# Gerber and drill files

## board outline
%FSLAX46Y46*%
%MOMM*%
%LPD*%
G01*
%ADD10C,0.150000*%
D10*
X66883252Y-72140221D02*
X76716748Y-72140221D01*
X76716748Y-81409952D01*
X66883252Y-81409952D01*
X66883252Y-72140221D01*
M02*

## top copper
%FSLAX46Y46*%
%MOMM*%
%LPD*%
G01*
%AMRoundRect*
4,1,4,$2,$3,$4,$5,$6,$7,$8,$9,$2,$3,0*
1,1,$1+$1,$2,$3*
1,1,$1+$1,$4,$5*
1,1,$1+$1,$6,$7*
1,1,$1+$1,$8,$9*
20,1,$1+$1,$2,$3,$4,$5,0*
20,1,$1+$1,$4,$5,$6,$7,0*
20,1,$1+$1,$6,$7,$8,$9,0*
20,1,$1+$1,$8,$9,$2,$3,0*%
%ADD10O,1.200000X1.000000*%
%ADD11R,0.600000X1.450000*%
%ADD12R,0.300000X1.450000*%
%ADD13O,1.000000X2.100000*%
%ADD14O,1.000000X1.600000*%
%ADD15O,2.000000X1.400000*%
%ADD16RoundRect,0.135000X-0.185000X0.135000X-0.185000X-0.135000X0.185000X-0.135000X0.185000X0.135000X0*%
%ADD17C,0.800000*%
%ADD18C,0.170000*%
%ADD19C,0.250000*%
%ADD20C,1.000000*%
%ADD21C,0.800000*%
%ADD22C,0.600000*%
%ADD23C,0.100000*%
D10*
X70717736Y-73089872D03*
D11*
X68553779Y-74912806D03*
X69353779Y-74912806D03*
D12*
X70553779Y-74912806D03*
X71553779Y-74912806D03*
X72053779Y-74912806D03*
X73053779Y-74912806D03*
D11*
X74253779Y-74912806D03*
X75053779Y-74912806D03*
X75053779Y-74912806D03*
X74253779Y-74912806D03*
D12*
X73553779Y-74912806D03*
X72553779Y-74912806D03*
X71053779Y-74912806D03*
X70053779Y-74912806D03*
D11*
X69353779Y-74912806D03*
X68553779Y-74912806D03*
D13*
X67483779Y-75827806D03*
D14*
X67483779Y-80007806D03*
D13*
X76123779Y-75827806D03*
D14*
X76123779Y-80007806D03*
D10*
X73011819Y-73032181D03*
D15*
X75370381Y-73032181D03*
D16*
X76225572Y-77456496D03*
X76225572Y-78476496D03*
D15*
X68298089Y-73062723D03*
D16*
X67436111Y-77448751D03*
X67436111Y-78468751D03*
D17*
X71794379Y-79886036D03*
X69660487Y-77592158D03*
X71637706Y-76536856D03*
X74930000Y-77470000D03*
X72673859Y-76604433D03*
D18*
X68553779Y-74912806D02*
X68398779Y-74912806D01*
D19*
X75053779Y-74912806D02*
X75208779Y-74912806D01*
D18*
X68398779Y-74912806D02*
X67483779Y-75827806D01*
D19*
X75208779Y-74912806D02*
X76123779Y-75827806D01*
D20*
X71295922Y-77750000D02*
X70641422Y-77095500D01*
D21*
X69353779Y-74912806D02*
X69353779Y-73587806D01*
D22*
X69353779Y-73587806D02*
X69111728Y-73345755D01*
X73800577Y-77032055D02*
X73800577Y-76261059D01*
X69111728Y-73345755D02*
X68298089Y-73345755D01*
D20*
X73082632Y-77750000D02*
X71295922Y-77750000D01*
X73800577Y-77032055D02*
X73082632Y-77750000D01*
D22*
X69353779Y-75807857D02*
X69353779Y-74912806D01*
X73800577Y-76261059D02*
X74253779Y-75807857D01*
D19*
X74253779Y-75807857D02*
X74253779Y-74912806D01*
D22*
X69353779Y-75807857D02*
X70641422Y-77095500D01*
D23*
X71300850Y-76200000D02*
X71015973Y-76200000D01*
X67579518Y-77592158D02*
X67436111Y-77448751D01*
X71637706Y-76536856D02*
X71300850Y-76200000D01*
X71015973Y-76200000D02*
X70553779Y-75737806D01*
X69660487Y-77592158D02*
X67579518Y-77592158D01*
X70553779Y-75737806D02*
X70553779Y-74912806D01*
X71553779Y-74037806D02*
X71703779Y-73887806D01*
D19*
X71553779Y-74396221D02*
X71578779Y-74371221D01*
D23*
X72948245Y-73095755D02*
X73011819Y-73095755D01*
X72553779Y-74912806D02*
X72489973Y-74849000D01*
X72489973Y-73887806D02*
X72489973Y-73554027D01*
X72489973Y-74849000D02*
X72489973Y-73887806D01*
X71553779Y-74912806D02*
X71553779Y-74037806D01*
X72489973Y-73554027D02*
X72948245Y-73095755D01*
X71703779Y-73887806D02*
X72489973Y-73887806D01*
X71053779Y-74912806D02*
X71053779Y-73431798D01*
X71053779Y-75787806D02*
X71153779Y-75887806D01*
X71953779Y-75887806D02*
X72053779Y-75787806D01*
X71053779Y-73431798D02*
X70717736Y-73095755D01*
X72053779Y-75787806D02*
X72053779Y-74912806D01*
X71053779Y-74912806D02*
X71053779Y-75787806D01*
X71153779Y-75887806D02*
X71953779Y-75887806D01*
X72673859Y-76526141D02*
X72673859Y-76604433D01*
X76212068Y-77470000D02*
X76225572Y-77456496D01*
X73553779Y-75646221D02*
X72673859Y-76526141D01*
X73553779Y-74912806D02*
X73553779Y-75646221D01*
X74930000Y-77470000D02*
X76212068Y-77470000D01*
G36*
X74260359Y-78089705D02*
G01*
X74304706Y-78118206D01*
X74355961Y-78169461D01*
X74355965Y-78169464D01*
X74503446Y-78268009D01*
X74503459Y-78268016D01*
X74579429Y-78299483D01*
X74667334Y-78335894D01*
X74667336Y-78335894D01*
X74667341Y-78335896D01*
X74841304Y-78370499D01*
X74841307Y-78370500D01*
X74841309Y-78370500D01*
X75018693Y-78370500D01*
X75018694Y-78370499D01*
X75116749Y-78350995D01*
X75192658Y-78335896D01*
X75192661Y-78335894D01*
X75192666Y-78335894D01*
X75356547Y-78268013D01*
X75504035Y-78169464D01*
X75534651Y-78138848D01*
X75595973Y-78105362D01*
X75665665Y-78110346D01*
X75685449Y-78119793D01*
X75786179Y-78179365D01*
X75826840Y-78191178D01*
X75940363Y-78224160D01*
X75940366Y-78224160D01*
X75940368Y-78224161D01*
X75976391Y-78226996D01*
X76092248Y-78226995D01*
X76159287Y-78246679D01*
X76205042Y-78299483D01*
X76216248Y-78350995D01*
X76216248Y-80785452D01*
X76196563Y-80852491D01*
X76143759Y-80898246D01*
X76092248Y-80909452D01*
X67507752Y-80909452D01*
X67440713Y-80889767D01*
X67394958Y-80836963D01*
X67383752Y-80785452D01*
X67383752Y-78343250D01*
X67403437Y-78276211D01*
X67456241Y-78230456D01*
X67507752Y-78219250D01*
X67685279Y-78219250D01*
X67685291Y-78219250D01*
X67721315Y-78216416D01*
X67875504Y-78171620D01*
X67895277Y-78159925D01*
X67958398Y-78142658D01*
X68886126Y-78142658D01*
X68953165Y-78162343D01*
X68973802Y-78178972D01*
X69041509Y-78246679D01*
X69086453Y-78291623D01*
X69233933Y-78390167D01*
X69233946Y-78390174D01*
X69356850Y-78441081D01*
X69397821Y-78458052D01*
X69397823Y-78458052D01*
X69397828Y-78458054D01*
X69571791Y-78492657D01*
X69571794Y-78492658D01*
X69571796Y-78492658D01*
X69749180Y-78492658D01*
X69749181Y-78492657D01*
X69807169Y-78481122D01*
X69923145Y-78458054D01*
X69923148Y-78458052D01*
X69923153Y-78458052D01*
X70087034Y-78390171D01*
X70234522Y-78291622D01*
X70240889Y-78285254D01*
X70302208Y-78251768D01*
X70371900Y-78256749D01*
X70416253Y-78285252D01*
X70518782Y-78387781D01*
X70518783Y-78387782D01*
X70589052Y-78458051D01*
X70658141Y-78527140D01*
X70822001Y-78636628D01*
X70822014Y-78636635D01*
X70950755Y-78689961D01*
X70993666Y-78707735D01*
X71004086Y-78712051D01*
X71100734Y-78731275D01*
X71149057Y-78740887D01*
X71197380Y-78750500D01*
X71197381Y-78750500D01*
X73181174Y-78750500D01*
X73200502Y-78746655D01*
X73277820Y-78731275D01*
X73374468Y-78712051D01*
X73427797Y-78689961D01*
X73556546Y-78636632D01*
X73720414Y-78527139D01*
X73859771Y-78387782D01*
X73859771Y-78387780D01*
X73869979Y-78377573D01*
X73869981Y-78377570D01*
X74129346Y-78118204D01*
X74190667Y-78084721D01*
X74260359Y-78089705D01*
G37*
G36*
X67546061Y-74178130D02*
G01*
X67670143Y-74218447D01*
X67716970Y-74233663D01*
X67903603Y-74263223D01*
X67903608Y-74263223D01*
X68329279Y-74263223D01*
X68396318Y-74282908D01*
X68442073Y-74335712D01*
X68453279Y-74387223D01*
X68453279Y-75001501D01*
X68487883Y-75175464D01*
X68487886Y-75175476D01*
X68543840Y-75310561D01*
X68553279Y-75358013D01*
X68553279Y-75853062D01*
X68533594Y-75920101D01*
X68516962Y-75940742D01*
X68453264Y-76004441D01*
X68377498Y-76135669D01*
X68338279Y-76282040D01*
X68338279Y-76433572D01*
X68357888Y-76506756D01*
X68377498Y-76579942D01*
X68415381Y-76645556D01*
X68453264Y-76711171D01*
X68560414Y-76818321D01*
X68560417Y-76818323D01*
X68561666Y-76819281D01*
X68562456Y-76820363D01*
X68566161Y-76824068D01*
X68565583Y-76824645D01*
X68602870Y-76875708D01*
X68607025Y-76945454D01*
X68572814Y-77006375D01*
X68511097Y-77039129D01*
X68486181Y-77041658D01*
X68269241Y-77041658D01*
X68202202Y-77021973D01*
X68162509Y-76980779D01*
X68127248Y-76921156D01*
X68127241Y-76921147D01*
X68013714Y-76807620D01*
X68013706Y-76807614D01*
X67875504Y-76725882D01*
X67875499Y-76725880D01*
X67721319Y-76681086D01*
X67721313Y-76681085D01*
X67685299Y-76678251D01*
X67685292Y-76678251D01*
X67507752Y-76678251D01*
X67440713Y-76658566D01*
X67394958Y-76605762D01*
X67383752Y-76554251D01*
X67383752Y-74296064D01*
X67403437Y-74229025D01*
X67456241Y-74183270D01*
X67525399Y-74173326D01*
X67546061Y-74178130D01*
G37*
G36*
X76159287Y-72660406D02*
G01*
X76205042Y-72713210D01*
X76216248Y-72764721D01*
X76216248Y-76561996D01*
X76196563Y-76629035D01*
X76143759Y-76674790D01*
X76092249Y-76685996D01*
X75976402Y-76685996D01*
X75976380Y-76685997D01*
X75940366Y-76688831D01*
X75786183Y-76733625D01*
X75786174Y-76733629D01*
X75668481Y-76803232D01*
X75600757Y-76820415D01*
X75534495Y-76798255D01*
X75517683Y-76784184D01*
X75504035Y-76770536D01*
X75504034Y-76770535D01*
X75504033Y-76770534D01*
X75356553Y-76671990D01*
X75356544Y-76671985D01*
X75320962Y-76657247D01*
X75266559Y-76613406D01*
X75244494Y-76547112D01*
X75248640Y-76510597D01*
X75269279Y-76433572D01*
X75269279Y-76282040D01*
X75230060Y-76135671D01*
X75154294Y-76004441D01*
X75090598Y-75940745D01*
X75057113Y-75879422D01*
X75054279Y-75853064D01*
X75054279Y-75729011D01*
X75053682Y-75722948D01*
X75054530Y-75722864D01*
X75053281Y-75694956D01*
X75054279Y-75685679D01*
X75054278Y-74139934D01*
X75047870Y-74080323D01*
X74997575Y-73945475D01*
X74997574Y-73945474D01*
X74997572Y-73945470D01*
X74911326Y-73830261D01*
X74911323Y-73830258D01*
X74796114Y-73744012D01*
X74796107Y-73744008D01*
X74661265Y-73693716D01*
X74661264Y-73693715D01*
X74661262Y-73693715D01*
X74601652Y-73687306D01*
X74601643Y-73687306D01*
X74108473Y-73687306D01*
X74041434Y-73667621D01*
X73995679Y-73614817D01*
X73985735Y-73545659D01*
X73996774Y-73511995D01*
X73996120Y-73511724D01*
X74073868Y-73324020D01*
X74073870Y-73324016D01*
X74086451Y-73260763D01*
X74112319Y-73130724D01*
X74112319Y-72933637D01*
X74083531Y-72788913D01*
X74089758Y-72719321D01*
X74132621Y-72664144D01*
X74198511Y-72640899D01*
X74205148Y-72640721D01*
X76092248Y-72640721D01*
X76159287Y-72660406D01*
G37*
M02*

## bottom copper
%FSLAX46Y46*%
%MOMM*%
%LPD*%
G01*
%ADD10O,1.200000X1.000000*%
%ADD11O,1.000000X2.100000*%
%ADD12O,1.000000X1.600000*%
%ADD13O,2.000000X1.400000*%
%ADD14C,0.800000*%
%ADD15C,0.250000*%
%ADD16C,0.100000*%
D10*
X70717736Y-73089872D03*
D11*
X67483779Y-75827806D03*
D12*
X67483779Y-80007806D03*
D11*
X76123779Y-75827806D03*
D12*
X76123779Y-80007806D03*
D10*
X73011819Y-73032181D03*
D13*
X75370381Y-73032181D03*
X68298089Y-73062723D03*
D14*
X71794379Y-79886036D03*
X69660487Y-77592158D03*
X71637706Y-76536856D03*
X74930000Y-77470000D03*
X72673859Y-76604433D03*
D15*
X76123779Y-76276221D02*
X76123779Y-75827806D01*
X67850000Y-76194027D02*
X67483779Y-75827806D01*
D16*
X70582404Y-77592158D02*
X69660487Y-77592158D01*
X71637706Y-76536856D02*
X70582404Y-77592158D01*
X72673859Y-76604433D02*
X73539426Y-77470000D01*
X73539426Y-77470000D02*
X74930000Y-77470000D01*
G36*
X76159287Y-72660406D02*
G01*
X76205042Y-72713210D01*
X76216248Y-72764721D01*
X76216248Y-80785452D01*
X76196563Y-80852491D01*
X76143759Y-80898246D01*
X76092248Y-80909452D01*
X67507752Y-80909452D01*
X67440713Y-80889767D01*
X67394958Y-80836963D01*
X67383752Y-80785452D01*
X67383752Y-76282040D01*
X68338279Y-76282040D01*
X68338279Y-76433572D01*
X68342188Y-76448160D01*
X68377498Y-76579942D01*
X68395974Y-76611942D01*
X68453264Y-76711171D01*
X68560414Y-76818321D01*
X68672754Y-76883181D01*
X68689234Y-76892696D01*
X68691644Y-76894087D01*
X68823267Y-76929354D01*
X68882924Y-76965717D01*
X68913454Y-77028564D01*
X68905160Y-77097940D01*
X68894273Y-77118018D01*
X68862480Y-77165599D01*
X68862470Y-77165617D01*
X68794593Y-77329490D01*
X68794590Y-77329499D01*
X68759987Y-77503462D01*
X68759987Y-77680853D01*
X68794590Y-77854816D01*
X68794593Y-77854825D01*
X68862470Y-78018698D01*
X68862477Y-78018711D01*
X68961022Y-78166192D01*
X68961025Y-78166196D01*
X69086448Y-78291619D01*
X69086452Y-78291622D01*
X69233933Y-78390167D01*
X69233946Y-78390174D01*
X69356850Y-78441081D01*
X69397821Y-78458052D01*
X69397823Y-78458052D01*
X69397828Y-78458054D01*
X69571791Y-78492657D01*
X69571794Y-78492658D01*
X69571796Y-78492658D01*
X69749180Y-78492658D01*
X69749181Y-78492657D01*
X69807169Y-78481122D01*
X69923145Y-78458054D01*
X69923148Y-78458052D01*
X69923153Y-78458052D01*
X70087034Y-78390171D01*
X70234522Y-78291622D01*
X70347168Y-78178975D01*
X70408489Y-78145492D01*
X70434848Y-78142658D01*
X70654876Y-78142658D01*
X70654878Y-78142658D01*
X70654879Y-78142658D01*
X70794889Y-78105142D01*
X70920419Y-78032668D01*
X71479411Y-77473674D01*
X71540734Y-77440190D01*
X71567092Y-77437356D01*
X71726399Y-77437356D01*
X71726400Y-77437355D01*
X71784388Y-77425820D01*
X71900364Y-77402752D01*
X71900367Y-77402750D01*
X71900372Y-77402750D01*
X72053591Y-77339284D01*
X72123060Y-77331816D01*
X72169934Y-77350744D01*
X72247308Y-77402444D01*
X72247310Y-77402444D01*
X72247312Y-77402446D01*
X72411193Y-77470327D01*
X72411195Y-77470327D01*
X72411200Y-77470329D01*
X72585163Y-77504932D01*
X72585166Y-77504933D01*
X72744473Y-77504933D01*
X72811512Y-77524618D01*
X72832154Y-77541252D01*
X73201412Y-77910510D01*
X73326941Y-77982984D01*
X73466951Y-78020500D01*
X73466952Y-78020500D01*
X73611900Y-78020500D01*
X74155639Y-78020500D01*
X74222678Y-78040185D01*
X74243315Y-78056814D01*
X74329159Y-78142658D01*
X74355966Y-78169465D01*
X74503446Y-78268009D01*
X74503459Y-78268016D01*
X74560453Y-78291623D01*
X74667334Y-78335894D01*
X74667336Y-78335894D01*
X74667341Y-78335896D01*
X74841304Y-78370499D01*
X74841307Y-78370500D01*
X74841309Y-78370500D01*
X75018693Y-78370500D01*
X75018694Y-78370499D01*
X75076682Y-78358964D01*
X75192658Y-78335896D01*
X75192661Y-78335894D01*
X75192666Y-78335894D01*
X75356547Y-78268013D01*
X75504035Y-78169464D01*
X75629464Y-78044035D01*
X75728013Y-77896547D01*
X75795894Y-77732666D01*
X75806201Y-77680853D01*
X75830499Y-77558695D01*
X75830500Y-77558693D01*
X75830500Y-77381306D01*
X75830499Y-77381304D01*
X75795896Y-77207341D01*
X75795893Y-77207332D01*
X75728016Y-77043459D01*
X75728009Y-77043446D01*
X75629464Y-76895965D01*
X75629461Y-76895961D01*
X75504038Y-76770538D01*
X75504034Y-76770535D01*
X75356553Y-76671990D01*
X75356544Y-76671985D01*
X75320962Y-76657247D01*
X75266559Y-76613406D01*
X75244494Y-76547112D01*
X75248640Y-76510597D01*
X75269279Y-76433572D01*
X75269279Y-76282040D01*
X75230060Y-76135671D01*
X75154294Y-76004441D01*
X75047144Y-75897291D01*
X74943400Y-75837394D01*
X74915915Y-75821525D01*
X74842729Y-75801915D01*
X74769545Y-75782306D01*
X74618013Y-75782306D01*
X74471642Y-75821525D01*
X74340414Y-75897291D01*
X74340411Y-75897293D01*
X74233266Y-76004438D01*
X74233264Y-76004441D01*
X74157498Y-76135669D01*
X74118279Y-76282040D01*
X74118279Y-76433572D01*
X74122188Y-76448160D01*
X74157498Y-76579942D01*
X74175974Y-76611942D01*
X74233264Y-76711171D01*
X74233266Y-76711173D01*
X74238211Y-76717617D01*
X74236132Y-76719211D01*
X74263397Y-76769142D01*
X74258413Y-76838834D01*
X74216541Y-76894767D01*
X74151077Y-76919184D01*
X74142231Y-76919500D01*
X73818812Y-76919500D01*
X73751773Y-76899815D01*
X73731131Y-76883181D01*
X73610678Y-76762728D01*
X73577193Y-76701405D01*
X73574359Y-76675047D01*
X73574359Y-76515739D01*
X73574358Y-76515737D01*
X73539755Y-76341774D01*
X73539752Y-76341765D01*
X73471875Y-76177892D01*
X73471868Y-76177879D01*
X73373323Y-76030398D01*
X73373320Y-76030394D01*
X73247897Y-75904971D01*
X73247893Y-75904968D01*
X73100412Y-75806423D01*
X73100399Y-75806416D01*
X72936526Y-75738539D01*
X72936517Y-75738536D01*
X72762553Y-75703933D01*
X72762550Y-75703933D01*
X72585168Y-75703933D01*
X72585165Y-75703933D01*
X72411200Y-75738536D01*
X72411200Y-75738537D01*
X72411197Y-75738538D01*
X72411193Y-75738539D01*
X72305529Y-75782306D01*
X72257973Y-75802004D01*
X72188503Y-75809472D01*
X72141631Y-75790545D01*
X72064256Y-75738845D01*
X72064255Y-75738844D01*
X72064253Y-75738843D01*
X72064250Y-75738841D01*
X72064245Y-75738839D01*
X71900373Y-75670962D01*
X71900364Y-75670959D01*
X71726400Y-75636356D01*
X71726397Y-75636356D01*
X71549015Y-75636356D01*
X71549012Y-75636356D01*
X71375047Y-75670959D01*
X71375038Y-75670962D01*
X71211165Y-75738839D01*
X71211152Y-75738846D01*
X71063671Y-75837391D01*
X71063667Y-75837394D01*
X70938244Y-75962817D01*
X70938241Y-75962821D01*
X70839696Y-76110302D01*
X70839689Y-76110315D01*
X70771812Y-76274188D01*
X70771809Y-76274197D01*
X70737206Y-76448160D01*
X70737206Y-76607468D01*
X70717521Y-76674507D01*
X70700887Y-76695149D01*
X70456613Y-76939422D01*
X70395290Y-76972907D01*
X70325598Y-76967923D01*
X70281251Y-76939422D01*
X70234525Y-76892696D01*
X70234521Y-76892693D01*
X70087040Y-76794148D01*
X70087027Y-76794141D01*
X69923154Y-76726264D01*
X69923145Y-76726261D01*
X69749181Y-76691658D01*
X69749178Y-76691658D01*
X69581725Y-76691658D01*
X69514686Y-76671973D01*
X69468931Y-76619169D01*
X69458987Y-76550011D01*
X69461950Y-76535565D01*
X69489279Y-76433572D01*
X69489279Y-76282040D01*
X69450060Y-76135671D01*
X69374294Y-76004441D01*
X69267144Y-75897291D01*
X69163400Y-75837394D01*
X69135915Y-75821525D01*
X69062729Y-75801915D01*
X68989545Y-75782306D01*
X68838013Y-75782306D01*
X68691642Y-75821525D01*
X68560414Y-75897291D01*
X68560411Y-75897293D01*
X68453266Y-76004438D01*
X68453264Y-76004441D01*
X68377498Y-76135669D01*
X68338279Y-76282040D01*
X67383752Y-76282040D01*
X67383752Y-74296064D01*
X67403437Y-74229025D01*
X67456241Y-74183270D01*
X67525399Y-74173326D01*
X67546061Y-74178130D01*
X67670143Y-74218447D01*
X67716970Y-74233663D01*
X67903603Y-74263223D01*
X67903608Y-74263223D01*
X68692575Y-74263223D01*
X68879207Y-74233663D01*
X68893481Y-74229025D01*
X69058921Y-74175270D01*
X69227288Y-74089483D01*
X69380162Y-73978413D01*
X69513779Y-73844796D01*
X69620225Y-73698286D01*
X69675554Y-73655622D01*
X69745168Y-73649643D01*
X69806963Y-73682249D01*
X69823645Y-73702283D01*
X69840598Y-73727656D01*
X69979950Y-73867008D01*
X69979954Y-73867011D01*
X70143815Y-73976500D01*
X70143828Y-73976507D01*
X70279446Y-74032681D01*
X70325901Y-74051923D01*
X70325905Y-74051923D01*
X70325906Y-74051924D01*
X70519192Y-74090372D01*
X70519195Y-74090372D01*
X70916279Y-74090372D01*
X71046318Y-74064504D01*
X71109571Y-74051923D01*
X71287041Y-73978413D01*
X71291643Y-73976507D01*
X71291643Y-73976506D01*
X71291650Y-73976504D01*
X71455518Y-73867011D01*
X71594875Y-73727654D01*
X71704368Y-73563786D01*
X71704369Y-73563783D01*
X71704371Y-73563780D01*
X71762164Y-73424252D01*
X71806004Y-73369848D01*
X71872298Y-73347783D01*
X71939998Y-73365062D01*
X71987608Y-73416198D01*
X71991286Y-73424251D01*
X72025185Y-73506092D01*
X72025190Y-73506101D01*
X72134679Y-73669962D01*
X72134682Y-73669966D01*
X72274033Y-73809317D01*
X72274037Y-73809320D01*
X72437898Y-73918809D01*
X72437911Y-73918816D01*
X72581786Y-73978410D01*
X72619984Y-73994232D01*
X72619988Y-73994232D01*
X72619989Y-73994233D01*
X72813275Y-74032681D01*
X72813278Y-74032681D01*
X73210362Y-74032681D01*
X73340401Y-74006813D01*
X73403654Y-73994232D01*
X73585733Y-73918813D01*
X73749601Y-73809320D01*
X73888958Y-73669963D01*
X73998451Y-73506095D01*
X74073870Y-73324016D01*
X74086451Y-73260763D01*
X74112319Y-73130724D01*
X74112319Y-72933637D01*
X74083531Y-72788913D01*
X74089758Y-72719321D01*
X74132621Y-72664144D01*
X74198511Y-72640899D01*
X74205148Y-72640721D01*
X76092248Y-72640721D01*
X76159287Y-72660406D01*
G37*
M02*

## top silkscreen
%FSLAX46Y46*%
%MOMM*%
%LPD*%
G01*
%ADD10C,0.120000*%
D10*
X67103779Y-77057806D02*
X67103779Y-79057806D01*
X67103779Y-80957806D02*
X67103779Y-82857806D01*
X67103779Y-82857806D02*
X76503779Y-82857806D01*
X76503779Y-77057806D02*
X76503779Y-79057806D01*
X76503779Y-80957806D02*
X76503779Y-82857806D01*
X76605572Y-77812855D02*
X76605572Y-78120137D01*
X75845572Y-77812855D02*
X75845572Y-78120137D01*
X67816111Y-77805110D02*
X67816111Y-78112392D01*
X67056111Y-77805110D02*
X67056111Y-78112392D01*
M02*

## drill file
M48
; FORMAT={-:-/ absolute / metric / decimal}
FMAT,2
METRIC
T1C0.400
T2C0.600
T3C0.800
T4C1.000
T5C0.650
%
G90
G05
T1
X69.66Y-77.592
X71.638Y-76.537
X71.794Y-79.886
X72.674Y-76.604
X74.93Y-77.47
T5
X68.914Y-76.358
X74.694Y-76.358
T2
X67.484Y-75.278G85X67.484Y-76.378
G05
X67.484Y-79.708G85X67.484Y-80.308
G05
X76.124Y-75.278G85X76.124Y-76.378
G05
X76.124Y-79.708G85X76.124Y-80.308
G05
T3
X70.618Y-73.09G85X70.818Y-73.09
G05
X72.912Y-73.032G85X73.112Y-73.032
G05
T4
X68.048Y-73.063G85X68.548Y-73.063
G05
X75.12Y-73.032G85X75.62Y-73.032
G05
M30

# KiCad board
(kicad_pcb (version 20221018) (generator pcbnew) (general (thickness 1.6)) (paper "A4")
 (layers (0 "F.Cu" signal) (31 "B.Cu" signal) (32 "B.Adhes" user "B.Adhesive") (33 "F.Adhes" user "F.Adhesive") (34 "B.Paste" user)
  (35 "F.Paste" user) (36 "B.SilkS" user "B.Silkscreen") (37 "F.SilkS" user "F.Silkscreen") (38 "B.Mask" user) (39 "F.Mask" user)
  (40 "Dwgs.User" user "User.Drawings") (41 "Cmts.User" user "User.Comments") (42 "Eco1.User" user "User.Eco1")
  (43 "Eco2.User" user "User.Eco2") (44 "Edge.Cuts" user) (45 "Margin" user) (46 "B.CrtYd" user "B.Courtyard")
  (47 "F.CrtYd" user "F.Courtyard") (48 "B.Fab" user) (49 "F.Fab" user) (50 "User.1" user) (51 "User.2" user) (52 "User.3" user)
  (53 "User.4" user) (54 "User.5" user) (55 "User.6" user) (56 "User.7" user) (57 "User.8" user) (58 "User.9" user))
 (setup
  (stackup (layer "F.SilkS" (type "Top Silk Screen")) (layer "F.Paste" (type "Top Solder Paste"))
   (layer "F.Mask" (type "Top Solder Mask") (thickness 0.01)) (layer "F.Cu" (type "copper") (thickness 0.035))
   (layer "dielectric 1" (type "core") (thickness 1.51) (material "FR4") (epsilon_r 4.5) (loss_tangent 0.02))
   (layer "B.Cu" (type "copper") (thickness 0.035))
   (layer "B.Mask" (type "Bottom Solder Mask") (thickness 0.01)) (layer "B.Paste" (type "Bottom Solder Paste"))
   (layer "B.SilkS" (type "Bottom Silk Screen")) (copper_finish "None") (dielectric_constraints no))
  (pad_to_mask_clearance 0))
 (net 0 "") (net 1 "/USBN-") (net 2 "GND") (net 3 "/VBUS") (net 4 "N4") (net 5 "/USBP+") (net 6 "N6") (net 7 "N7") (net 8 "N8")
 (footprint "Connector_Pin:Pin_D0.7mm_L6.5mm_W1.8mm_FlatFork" (layer "F.Cu") (at 70.717736 73.089872)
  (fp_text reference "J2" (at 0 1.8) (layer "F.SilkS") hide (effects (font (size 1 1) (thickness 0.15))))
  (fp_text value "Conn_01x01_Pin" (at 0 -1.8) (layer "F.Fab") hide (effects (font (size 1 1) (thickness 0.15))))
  (pad "1" thru_hole oval (at 0 0) (size 1.2 1) (drill oval 1 0.8) (layers "*.Cu" "*.Mask") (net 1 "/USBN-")))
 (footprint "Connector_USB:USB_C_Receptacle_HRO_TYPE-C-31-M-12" (layer "F.Cu") (at 71.803779 78.957806)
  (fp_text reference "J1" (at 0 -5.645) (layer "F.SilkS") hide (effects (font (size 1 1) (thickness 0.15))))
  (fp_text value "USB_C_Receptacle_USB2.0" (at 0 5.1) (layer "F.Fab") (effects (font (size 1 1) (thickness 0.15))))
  (fp_line (start -4.7 -1.9) (end -4.7 0.1) (stroke (width 0.12) (type solid)) (layer "F.SilkS"))
  (fp_line (start -4.7 2) (end -4.7 3.9) (stroke (width 0.12) (type solid)) (layer "F.SilkS"))
  (fp_line (start -4.7 3.9) (end 4.7 3.9) (stroke (width 0.12) (type solid)) (layer "F.SilkS"))
  (fp_line (start 4.7 -1.9) (end 4.7 0.1) (stroke (width 0.12) (type solid)) (layer "F.SilkS"))
  (fp_line (start 4.7 2) (end 4.7 3.9) (stroke (width 0.12) (type solid)) (layer "F.SilkS"))
  (pad "" np_thru_hole circle (at -2.89 -2.6) (size 0.65 0.65) (drill 0.65) (layers "*.Cu" "*.Mask"))
  (pad "" np_thru_hole circle (at 2.89 -2.6) (size 0.65 0.65) (drill 0.65) (layers "*.Cu" "*.Mask"))
  (pad "A1" smd rect (at -3.25 -4.045) (size 0.6 1.45) (layers "F.Cu" "F.Paste" "F.Mask") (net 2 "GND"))
  (pad "A4" smd rect (at -2.45 -4.045) (size 0.6 1.45) (layers "F.Cu" "F.Paste" "F.Mask") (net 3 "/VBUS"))
  (pad "A5" smd rect (at -1.25 -4.045) (size 0.3 1.45) (layers "F.Cu" "F.Paste" "F.Mask") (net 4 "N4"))
  (pad "A6" smd rect (at -0.25 -4.045) (size 0.3 1.45) (layers "F.Cu" "F.Paste" "F.Mask") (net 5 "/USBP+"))
  (pad "A7" smd rect (at 0.25 -4.045) (size 0.3 1.45) (layers "F.Cu" "F.Paste" "F.Mask") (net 1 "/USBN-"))
  (pad "A8" smd rect (at 1.25 -4.045) (size 0.3 1.45) (layers "F.Cu" "F.Paste" "F.Mask") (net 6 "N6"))
  (pad "A9" smd rect (at 2.45 -4.045) (size 0.6 1.45) (layers "F.Cu" "F.Paste" "F.Mask") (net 3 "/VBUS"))
  (pad "A12" smd rect (at 3.25 -4.045) (size 0.6 1.45) (layers "F.Cu" "F.Paste" "F.Mask") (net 2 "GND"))
  (pad "B1" smd rect (at 3.25 -4.045) (size 0.6 1.45) (layers "F.Cu" "F.Paste" "F.Mask") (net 2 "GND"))
  (pad "B4" smd rect (at 2.45 -4.045) (size 0.6 1.45) (layers "F.Cu" "F.Paste" "F.Mask") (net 3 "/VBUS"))
  (pad "B5" smd rect (at 1.75 -4.045) (size 0.3 1.45) (layers "F.Cu" "F.Paste" "F.Mask") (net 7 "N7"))
  (pad "B6" smd rect (at 0.75 -4.045) (size 0.3 1.45) (layers "F.Cu" "F.Paste" "F.Mask") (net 5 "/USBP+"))
  (pad "B7" smd rect (at -0.75 -4.045) (size 0.3 1.45) (layers "F.Cu" "F.Paste" "F.Mask") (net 1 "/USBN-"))
  (pad "B8" smd rect (at -1.75 -4.045) (size 0.3 1.45) (layers "F.Cu" "F.Paste" "F.Mask") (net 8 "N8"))
  (pad "B9" smd rect (at -2.45 -4.045) (size 0.6 1.45) (layers "F.Cu" "F.Paste" "F.Mask") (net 3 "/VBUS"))
  (pad "B12" smd rect (at -3.25 -4.045) (size 0.6 1.45) (layers "F.Cu" "F.Paste" "F.Mask") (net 2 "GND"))
  (pad "S1" thru_hole oval (at -4.32 -3.13) (size 1 2.1) (drill oval 0.6 1.7) (layers "*.Cu" "*.Mask") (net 2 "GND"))
  (pad "S1" thru_hole oval (at -4.32 1.05) (size 1 1.6) (drill oval 0.6 1.2) (layers "*.Cu" "*.Mask") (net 2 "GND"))
  (pad "S1" thru_hole oval (at 4.32 -3.13) (size 1 2.1) (drill oval 0.6 1.7) (layers "*.Cu" "*.Mask") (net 2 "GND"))
  (pad "S1" thru_hole oval (at 4.32 1.05) (size 1 1.6) (drill oval 0.6 1.2) (layers "*.Cu" "*.Mask") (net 2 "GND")))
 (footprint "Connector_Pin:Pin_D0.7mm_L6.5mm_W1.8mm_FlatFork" (layer "F.Cu") (at 73.011819 73.032181)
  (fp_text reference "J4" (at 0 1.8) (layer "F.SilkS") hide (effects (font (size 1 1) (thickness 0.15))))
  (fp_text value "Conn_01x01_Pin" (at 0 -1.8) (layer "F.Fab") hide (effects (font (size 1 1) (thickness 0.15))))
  (pad "1" thru_hole oval (at 0 0) (size 1.2 1) (drill oval 1 0.8) (layers "*.Cu" "*.Mask") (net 5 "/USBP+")))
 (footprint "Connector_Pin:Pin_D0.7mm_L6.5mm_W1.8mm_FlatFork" (layer "F.Cu") (at 75.370381 73.032181)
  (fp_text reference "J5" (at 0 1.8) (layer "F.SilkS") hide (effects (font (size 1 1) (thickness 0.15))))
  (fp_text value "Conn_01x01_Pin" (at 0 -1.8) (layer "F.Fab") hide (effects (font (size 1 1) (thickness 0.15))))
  (pad "1" thru_hole oval (at 0 0) (size 2 1.4) (drill oval 1.5 1) (layers "*.Cu" "*.Mask") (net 2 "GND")))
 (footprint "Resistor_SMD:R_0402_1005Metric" (layer "F.Cu") (at 76.225572 77.966496 -90)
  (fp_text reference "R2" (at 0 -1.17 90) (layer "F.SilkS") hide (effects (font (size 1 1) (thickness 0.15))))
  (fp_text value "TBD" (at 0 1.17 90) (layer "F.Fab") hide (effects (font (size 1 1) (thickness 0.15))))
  (fp_line (start -0.153641 -0.38) (end 0.153641 -0.38) (stroke (width 0.12) (type solid)) (layer "F.SilkS"))
  (fp_line (start -0.153641 0.38) (end 0.153641 0.38) (stroke (width 0.12) (type solid)) (layer "F.SilkS"))
  (pad "1" smd roundrect (at -0.51 0 270) (size 0.54 0.64) (layers "F.Cu" "F.Paste" "F.Mask") (roundrect_rratio 0.25) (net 7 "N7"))
  (pad "2" smd roundrect (at 0.51 0 270) (size 0.54 0.64) (layers "F.Cu" "F.Paste" "F.Mask") (roundrect_rratio 0.25) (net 2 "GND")))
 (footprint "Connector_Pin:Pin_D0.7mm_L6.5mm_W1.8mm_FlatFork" (layer "F.Cu") (at 68.298089 73.062723)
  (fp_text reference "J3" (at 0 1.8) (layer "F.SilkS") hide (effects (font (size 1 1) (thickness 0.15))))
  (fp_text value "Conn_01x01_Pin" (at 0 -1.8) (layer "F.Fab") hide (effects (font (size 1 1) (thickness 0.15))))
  (pad "1" thru_hole oval (at 0 0) (size 2 1.4) (drill oval 1.5 1) (layers "*.Cu" "*.Mask") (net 3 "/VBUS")))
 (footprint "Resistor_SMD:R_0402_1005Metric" (layer "F.Cu") (at 67.436111 77.958751 -90)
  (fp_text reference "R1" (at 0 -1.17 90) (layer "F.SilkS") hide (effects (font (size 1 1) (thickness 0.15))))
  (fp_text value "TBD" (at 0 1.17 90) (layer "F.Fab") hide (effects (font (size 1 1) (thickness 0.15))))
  (fp_line (start -0.153641 -0.38) (end 0.153641 -0.38) (stroke (width 0.12) (type solid)) (layer "F.SilkS"))
  (fp_line (start -0.153641 0.38) (end 0.153641 0.38) (stroke (width 0.12) (type solid)) (layer "F.SilkS"))
  (pad "1" smd roundrect (at -0.51 0 270) (size 0.54 0.64) (layers "F.Cu" "F.Paste" "F.Mask") (roundrect_rratio 0.25) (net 4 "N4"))
  (pad "2" smd roundrect (at 0.51 0 270) (size 0.54 0.64) (layers "F.Cu" "F.Paste" "F.Mask") (roundrect_rratio 0.25) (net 2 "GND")))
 (gr_rect (start 66.883252 72.140221) (end 76.716748 81.409952) (stroke (width 0.15) (type default)) (fill none) (layer "Edge.Cuts"))
 (segment (start 68.553779 74.912806) (end 68.398779 74.912806) (width 0.17) (layer "F.Cu") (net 2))
 (segment (start 75.053779 74.912806) (end 75.208779 74.912806) (width 0.25) (layer "F.Cu") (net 2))
 (segment (start 68.398779 74.912806) (end 67.483779 75.827806) (width 0.17) (layer "F.Cu") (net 2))
 (segment (start 75.208779 74.912806) (end 76.123779 75.827806) (width 0.25) (layer "F.Cu") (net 2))
 (via (at 71.794379 79.886036) (size 0.8) (drill 0.4) (layers "F.Cu" "B.Cu") (free) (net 2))
 (segment (start 76.123779 76.276221) (end 76.123779 75.827806) (width 0.25) (layer "B.Cu") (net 2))
 (segment (start 67.85 76.194027) (end 67.483779 75.827806) (width 0.25) (layer "B.Cu") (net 2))
 (segment (start 71.295922 77.75) (end 70.641422 77.0955) (width 1) (layer "F.Cu") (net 3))
 (segment (start 69.353779 74.912806) (end 69.353779 73.587806) (width 0.8) (layer "F.Cu") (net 3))
 (segment (start 69.353779 73.587806) (end 69.111728 73.345755) (width 0.6) (layer "F.Cu") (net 3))
 (segment (start 73.800577 77.032055) (end 73.800577 76.261059) (width 0.6) (layer "F.Cu") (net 3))
 (segment (start 69.111728 73.345755) (end 68.298089 73.345755) (width 0.6) (layer "F.Cu") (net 3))
 (segment (start 73.082632 77.75) (end 71.295922 77.75) (width 1) (layer "F.Cu") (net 3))
 (segment (start 73.800577 77.032055) (end 73.082632 77.75) (width 1) (layer "F.Cu") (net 3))
 (segment (start 69.353779 75.807857) (end 69.353779 74.912806) (width 0.6) (layer "F.Cu") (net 3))
 (segment (start 73.800577 76.261059) (end 74.253779 75.807857) (width 0.6) (layer "F.Cu") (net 3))
 (segment (start 74.253779 75.807857) (end 74.253779 74.912806) (width 0.25) (layer "F.Cu") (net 3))
 (segment (start 69.353779 75.807857) (end 70.641422 77.0955) (width 0.6) (layer "F.Cu") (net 3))
 (segment (start 71.30085 76.2) (end 71.015973 76.2) (width 0.1) (layer "F.Cu") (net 4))
 (segment (start 67.579518 77.592158) (end 67.436111 77.448751) (width 0.1) (layer "F.Cu") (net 4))
 (segment (start 71.637706 76.536856) (end 71.30085 76.2) (width 0.1) (layer "F.Cu") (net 4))
 (segment (start 71.015973 76.2) (end 70.553779 75.737806) (width 0.1) (layer "F.Cu") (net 4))
 (segment (start 69.660487 77.592158) (end 67.579518 77.592158) (width 0.1) (layer "F.Cu") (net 4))
 (segment (start 70.553779 75.737806) (end 70.553779 74.912806) (width 0.1) (layer "F.Cu") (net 4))
 (via (at 69.660487 77.592158) (size 0.8) (drill 0.4) (layers "F.Cu" "B.Cu") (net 4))
 (via (at 71.637706 76.536856) (size 0.8) (drill 0.4) (layers "F.Cu" "B.Cu") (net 4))
 (segment (start 70.582404 77.592158) (end 69.660487 77.592158) (width 0.1) (layer "B.Cu") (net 4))
 (segment (start 71.637706 76.536856) (end 70.582404 77.592158) (width 0.1) (layer "B.Cu") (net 4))
 (segment (start 71.553779 74.037806) (end 71.703779 73.887806) (width 0.1) (layer "F.Cu") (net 5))
 (segment (start 71.553779 74.396221) (end 71.578779 74.371221) (width 0.25) (layer "F.Cu") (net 5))
 (segment (start 72.948245 73.095755) (end 73.011819 73.095755) (width 0.1) (layer "F.Cu") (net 5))
 (segment (start 72.553779 74.912806) (end 72.489973 74.849) (width 0.1) (layer "F.Cu") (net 5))
 (segment (start 72.489973 73.887806) (end 72.489973 73.554027) (width 0.1) (layer "F.Cu") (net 5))
 (segment (start 72.489973 74.849) (end 72.489973 73.887806) (width 0.1) (layer "F.Cu") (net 5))
 (segment (start 71.553779 74.912806) (end 71.553779 74.037806) (width 0.1) (layer "F.Cu") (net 5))
 (segment (start 72.489973 73.554027) (end 72.948245 73.095755) (width 0.1) (layer "F.Cu") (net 5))
 (segment (start 71.703779 73.887806) (end 72.489973 73.887806) (width 0.1) (layer "F.Cu") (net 5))
 (segment (start 71.053779 74.912806) (end 71.053779 73.431798) (width 0.1) (layer "F.Cu") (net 1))
 (segment (start 71.053779 75.787806) (end 71.153779 75.887806) (width 0.1) (layer "F.Cu") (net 1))
 (segment (start 71.953779 75.887806) (end 72.053779 75.787806) (width 0.1) (layer "F.Cu") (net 1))
 (segment (start 71.053779 73.431798) (end 70.717736 73.095755) (width 0.1) (layer "F.Cu") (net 1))
 (segment (start 72.053779 75.787806) (end 72.053779 74.912806) (width 0.1) (layer "F.Cu") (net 1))
 (segment (start 71.053779 74.912806) (end 71.053779 75.787806) (width 0.1) (layer "F.Cu") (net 1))
 (segment (start 71.153779 75.887806) (end 71.953779 75.887806) (width 0.1) (layer "F.Cu") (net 1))
 (segment (start 72.673859 76.526141) (end 72.673859 76.604433) (width 0.1) (layer "F.Cu") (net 7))
 (segment (start 76.212068 77.47) (end 76.225572 77.456496) (width 0.1) (layer "F.Cu") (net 7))
 (segment (start 73.553779 75.646221) (end 72.673859 76.526141) (width 0.1) (layer "F.Cu") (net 7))
 (segment (start 73.553779 74.912806) (end 73.553779 75.646221) (width 0.1) (layer "F.Cu") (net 7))
 (segment (start 74.93 77.47) (end 76.212068 77.47) (width 0.1) (layer "F.Cu") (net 7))
 (via (at 74.93 77.47) (size 0.8) (drill 0.4) (layers "F.Cu" "B.Cu") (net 7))
 (via (at 72.673859 76.604433) (size 0.8) (drill 0.4) (layers "F.Cu" "B.Cu") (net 7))
 (segment (start 72.673859 76.604433) (end 73.539426 77.47) (width 0.1) (layer "B.Cu") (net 7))
 (segment (start 73.539426 77.47) (end 74.93 77.47) (width 0.1) (layer "B.Cu") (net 7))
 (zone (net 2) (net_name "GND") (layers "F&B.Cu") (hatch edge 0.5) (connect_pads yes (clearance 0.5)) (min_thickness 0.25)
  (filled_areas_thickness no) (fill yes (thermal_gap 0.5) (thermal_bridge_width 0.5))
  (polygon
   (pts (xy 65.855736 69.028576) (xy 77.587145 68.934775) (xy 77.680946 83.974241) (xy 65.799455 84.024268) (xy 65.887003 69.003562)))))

